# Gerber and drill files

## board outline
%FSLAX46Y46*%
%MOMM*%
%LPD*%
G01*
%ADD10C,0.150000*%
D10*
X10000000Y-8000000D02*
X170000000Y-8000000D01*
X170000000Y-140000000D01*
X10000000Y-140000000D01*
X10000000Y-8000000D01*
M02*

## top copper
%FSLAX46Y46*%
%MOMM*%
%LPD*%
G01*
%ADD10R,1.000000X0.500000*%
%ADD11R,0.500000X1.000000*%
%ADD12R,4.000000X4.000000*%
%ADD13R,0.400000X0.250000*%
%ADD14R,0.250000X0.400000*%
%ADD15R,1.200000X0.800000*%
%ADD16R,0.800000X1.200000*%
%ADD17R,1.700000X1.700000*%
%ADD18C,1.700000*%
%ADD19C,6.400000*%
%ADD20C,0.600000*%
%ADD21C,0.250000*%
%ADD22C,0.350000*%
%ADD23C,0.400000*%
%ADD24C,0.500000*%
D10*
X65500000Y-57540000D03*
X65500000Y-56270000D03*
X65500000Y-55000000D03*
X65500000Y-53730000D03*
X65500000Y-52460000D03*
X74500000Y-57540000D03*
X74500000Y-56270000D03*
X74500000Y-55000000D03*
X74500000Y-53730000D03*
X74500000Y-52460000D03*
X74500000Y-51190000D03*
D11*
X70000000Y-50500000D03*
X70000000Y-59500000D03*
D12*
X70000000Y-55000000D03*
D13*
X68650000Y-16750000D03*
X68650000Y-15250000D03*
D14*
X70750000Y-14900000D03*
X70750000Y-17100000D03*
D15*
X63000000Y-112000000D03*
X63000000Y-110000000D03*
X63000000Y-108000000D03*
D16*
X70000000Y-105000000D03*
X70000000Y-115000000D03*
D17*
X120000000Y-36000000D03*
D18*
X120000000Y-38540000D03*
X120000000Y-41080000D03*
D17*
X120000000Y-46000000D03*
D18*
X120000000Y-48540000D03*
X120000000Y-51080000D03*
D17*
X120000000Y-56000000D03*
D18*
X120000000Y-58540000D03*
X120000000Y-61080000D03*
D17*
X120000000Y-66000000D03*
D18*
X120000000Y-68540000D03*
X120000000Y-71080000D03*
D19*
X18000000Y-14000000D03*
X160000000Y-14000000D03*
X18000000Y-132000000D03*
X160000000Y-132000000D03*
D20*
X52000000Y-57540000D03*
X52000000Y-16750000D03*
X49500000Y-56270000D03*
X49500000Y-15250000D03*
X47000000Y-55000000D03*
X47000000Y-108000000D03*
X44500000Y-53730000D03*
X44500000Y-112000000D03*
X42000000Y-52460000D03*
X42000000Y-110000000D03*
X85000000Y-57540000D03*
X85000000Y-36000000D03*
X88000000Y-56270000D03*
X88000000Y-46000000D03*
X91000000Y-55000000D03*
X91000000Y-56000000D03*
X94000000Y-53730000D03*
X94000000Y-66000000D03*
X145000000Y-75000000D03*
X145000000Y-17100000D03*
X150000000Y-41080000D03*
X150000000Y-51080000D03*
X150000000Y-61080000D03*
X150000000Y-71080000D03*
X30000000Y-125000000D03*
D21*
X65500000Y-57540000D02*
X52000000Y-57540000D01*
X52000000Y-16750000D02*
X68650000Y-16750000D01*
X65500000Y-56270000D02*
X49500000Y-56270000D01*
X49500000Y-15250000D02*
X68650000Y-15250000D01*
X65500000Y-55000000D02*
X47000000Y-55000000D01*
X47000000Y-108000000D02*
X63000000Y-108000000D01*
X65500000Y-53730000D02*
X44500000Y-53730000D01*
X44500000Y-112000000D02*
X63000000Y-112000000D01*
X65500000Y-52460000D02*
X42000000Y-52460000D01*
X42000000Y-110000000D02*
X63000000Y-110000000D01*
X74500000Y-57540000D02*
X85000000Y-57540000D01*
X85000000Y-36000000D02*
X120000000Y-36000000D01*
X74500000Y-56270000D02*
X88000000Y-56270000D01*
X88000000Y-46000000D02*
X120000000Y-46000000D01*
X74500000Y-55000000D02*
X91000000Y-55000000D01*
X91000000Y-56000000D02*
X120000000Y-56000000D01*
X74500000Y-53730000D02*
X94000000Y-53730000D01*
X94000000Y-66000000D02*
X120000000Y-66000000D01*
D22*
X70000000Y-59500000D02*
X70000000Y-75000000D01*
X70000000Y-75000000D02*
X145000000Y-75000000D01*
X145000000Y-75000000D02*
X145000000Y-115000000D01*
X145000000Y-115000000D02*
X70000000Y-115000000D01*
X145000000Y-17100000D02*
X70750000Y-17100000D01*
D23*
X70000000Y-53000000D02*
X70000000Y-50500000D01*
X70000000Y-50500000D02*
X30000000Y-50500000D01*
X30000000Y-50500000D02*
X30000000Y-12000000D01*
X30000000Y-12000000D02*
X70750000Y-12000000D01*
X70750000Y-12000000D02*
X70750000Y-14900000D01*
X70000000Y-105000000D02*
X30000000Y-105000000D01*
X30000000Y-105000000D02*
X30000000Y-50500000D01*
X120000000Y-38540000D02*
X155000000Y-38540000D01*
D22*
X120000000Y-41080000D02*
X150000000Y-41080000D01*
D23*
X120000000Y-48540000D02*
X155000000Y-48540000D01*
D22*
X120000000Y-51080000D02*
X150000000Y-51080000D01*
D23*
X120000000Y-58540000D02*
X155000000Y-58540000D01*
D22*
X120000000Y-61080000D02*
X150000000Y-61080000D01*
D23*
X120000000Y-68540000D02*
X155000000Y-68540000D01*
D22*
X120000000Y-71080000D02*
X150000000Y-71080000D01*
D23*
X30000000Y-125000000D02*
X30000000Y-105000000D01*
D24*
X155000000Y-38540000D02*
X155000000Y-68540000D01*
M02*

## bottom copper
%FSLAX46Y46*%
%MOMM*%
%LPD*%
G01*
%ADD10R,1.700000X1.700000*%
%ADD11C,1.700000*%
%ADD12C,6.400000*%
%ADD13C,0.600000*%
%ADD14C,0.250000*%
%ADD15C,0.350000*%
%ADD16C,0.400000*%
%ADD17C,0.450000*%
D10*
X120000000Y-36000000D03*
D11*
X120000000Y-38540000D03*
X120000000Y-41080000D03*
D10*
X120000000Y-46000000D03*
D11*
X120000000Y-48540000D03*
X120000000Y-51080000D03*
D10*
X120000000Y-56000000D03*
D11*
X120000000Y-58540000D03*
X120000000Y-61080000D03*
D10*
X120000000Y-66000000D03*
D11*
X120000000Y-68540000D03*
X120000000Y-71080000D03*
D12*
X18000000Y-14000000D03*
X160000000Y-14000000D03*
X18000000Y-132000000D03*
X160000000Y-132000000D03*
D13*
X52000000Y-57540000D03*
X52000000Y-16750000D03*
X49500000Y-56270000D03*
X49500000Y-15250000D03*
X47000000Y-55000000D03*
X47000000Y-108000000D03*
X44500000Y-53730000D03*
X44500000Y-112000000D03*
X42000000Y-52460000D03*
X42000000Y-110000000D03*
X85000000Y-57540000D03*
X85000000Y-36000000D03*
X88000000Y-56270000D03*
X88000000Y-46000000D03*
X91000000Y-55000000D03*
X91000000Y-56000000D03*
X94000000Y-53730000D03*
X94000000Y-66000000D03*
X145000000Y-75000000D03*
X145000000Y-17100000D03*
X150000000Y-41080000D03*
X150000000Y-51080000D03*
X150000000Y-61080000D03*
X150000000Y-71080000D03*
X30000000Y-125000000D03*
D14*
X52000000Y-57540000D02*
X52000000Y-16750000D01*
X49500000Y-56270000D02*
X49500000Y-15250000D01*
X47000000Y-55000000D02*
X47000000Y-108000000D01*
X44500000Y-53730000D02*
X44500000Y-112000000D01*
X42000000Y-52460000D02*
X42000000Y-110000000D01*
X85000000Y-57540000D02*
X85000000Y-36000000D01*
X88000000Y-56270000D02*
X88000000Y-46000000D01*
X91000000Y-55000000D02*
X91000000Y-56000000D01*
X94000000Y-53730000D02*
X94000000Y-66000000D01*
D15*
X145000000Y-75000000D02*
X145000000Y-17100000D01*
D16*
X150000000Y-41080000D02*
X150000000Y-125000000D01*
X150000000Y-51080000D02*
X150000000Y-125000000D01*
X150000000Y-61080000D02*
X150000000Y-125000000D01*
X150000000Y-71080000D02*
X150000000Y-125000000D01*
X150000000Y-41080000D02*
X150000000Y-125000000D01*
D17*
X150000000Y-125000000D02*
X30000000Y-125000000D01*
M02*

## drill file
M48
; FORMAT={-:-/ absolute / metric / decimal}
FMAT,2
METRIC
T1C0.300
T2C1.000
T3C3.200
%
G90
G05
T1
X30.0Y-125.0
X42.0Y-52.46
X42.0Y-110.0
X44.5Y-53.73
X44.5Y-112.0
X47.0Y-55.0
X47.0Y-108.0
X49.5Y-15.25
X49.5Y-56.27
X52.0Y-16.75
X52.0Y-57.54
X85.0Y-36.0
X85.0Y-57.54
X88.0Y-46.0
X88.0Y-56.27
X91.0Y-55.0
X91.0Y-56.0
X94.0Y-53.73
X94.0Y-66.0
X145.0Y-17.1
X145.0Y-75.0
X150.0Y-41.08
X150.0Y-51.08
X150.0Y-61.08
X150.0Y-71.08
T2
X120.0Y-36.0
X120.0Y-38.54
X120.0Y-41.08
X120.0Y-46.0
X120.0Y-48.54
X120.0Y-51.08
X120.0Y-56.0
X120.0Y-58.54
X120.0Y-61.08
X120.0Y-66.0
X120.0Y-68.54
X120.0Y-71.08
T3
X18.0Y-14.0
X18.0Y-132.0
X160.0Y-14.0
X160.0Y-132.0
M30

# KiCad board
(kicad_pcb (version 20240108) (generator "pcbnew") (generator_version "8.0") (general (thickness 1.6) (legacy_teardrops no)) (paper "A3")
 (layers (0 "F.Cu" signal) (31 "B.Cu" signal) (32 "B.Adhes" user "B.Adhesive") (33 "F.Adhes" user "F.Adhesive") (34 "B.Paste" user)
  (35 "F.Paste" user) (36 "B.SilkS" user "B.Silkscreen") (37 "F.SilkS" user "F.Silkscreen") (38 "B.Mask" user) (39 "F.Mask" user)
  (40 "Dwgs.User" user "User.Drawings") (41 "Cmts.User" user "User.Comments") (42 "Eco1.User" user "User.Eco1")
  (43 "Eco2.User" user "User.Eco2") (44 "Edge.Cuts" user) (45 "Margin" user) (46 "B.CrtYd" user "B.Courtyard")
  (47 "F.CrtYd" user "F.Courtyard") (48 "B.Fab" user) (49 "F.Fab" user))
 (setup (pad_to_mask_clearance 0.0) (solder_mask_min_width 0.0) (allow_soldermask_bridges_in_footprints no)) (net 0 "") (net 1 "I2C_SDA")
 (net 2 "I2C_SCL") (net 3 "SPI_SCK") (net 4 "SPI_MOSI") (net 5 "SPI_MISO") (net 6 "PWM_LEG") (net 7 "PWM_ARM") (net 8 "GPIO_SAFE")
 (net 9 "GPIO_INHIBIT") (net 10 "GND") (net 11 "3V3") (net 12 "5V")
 (gr_rect (start 10 8) (end 170 140) (stroke (width 0.15) (type solid)) (fill none) (layer "Edge.Cuts"))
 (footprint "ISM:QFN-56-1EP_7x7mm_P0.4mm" (layer "F.Cu") (at 70 55)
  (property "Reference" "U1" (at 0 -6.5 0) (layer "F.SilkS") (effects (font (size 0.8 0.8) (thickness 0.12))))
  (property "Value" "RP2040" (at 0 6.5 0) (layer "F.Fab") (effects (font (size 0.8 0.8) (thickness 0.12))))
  (pad "1" smd rect (at -4.5 2.54) (size 1.0 0.5) (layers "F.Cu" "F.Paste" "F.Mask") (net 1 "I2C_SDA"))
  (pad "2" smd rect (at -4.5 1.27) (size 1.0 0.5) (layers "F.Cu" "F.Paste" "F.Mask") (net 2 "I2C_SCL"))
  (pad "3" smd rect (at -4.5 0) (size 1.0 0.5) (layers "F.Cu" "F.Paste" "F.Mask") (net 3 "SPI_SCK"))
  (pad "4" smd rect (at -4.5 -1.27) (size 1.0 0.5) (layers "F.Cu" "F.Paste" "F.Mask") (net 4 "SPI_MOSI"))
  (pad "5" smd rect (at -4.5 -2.54) (size 1.0 0.5) (layers "F.Cu" "F.Paste" "F.Mask") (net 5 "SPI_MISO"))
  (pad "6" smd rect (at 4.5 2.54) (size 1.0 0.5) (layers "F.Cu" "F.Paste" "F.Mask") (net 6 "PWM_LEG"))
  (pad "7" smd rect (at 4.5 1.27) (size 1.0 0.5) (layers "F.Cu" "F.Paste" "F.Mask") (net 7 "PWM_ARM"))
  (pad "8" smd rect (at 4.5 0) (size 1.0 0.5) (layers "F.Cu" "F.Paste" "F.Mask") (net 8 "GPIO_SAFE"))
  (pad "9" smd rect (at 4.5 -1.27) (size 1.0 0.5) (layers "F.Cu" "F.Paste" "F.Mask") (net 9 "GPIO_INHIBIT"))
  (pad "12" smd rect (at 4.5 -2.54) (size 1.0 0.5) (layers "F.Cu" "F.Paste" "F.Mask"))
  (pad "13" smd rect (at 4.5 -3.81) (size 1.0 0.5) (layers "F.Cu" "F.Paste" "F.Mask"))
  (pad "10" smd rect (at 0 -4.5) (size 0.5 1.0) (layers "F.Cu" "F.Paste" "F.Mask") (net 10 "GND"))
  (pad "11" smd rect (at 0 4.5) (size 0.5 1.0) (layers "F.Cu" "F.Paste" "F.Mask") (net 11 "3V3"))
  (pad "EP" smd rect (at 0 0) (size 4 4) (layers "F.Cu" "F.Paste" "F.Mask") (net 10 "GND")))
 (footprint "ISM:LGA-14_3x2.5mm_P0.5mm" (layer "F.Cu") (at 70 16)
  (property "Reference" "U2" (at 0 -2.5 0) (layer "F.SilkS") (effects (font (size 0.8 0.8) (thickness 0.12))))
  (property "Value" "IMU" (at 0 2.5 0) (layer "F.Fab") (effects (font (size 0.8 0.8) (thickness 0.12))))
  (pad "1" smd rect (at -1.35 0.75) (size 0.4 0.25) (layers "F.Cu" "F.Paste" "F.Mask") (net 1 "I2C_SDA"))
  (pad "2" smd rect (at -1.35 -0.75) (size 0.4 0.25) (layers "F.Cu" "F.Paste" "F.Mask") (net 2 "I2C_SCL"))
  (pad "3" smd rect (at 0.75 -1.1) (size 0.25 0.4) (layers "F.Cu" "F.Paste" "F.Mask") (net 10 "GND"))
  (pad "4" smd rect (at 0.75 1.1) (size 0.25 0.4) (layers "F.Cu" "F.Paste" "F.Mask") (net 11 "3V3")))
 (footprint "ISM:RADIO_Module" (layer "F.Cu") (at 70 110)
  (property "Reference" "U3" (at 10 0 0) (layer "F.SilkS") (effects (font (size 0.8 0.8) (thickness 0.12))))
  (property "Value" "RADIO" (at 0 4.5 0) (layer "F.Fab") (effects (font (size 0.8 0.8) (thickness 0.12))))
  (pad "1" smd rect (at -7 2) (size 1.2 0.8) (layers "F.Cu" "F.Paste" "F.Mask") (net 4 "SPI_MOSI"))
  (pad "2" smd rect (at -7 0) (size 1.2 0.8) (layers "F.Cu" "F.Paste" "F.Mask") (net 5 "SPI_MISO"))
  (pad "3" smd rect (at -7 -2) (size 1.2 0.8) (layers "F.Cu" "F.Paste" "F.Mask") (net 3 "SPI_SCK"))
  (pad "4" smd rect (at 0 -5) (size 0.8 1.2) (layers "F.Cu" "F.Paste" "F.Mask") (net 10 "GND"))
  (pad "5" smd rect (at 0 5) (size 0.8 1.2) (layers "F.Cu" "F.Paste" "F.Mask") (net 11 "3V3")))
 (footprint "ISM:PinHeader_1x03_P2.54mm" (layer "F.Cu") (at 120 36)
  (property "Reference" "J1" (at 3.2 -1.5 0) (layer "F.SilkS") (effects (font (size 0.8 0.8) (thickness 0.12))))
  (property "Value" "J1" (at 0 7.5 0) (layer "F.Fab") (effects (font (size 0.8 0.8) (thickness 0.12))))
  (pad "1" thru_hole rect (at 0 0) (size 1.7 1.7) (drill 1.0) (layers "*.Cu" "*.Mask") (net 6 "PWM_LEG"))
  (pad "2" thru_hole circle (at 0 2.54) (size 1.7 1.7) (drill 1.0) (layers "*.Cu" "*.Mask") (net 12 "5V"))
  (pad "3" thru_hole circle (at 0 5.08) (size 1.7 1.7) (drill 1.0) (layers "*.Cu" "*.Mask") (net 10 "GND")))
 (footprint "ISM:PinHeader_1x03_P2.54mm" (layer "F.Cu") (at 120 46)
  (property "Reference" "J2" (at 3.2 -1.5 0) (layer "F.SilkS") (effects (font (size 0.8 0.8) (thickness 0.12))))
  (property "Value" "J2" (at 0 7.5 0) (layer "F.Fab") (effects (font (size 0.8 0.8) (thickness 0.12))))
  (pad "1" thru_hole rect (at 0 0) (size 1.7 1.7) (drill 1.0) (layers "*.Cu" "*.Mask") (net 7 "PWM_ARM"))
  (pad "2" thru_hole circle (at 0 2.54) (size 1.7 1.7) (drill 1.0) (layers "*.Cu" "*.Mask") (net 12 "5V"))
  (pad "3" thru_hole circle (at 0 5.08) (size 1.7 1.7) (drill 1.0) (layers "*.Cu" "*.Mask") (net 10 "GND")))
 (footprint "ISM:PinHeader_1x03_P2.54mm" (layer "F.Cu") (at 120 56)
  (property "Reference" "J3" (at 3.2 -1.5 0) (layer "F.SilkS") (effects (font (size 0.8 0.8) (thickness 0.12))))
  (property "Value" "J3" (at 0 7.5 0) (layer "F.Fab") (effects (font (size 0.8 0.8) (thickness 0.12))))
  (pad "1" thru_hole rect (at 0 0) (size 1.7 1.7) (drill 1.0) (layers "*.Cu" "*.Mask") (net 8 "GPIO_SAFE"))
  (pad "2" thru_hole circle (at 0 2.54) (size 1.7 1.7) (drill 1.0) (layers "*.Cu" "*.Mask") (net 12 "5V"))
  (pad "3" thru_hole circle (at 0 5.08) (size 1.7 1.7) (drill 1.0) (layers "*.Cu" "*.Mask") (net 10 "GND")))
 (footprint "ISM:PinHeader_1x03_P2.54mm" (layer "F.Cu") (at 120 66)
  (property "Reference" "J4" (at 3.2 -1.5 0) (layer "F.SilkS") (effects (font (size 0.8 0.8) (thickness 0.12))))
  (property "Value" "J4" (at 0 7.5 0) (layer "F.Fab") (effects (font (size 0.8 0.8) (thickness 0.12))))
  (pad "1" thru_hole rect (at 0 0) (size 1.7 1.7) (drill 1.0) (layers "*.Cu" "*.Mask") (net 9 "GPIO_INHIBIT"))
  (pad "2" thru_hole circle (at 0 2.54) (size 1.7 1.7) (drill 1.0) (layers "*.Cu" "*.Mask") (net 12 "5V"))
  (pad "3" thru_hole circle (at 0 5.08) (size 1.7 1.7) (drill 1.0) (layers "*.Cu" "*.Mask") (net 10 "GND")))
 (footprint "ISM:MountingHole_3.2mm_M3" (layer "F.Cu") (at 18 14)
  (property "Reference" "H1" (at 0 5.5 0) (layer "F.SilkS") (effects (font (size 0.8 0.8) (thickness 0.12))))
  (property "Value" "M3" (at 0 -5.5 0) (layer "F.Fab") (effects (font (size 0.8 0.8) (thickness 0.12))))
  (pad "" thru_hole circle (at 0 0) (size 6.4 6.4) (drill 3.2) (layers "*.Cu" "*.Mask")))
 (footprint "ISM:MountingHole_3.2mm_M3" (layer "F.Cu") (at 160 14)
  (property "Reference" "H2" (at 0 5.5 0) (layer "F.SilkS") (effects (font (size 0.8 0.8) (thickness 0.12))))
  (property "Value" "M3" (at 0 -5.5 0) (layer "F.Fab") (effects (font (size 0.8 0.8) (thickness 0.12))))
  (pad "" thru_hole circle (at 0 0) (size 6.4 6.4) (drill 3.2) (layers "*.Cu" "*.Mask")))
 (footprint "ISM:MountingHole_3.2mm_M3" (layer "F.Cu") (at 18 132)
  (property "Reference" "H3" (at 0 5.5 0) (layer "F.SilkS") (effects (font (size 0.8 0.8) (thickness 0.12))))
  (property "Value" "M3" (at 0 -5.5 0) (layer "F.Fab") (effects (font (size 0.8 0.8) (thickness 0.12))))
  (pad "" thru_hole circle (at 0 0) (size 6.4 6.4) (drill 3.2) (layers "*.Cu" "*.Mask")))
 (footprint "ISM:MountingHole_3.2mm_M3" (layer "F.Cu") (at 160 132)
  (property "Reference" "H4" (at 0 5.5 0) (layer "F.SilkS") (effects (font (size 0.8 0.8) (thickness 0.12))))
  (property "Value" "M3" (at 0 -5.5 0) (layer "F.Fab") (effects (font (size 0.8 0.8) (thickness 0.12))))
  (pad "" thru_hole circle (at 0 0) (size 6.4 6.4) (drill 3.2) (layers "*.Cu" "*.Mask")))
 (segment (start 65.5 57.54) (end 52.0 57.54) (width 0.25) (layer "F.Cu") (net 1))
 (segment (start 52.0 57.54) (end 52.0 16.75) (width 0.25) (layer "B.Cu") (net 1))
 (segment (start 52.0 16.75) (end 68.65 16.75) (width 0.25) (layer "F.Cu") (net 1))
 (segment (start 65.5 56.27) (end 49.5 56.27) (width 0.25) (layer "F.Cu") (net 2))
 (segment (start 49.5 56.27) (end 49.5 15.25) (width 0.25) (layer "B.Cu") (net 2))
 (segment (start 49.5 15.25) (end 68.65 15.25) (width 0.25) (layer "F.Cu") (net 2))
 (segment (start 65.5 55) (end 47.0 55) (width 0.25) (layer "F.Cu") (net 3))
 (segment (start 47.0 55) (end 47.0 108) (width 0.25) (layer "B.Cu") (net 3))
 (segment (start 47.0 108) (end 63 108) (width 0.25) (layer "F.Cu") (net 3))
 (segment (start 65.5 53.73) (end 44.5 53.73) (width 0.25) (layer "F.Cu") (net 4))
 (segment (start 44.5 53.73) (end 44.5 112) (width 0.25) (layer "B.Cu") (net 4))
 (segment (start 44.5 112) (end 63 112) (width 0.25) (layer "F.Cu") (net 4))
 (segment (start 65.5 52.46) (end 42.0 52.46) (width 0.25) (layer "F.Cu") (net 5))
 (segment (start 42.0 52.46) (end 42.0 110) (width 0.25) (layer "B.Cu") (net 5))
 (segment (start 42.0 110) (end 63 110) (width 0.25) (layer "F.Cu") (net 5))
 (segment (start 74.5 57.54) (end 85 57.54) (width 0.25) (layer "F.Cu") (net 6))
 (segment (start 85 57.54) (end 85 36) (width 0.25) (layer "B.Cu") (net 6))
 (segment (start 85 36) (end 120 36) (width 0.25) (layer "F.Cu") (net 6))
 (segment (start 74.5 56.27) (end 88 56.27) (width 0.25) (layer "F.Cu") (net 7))
 (segment (start 88 56.27) (end 88 46) (width 0.25) (layer "B.Cu") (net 7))
 (segment (start 88 46) (end 120 46) (width 0.25) (layer "F.Cu") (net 7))
 (segment (start 74.5 55) (end 91 55) (width 0.25) (layer "F.Cu") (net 8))
 (segment (start 91 55) (end 91 56) (width 0.25) (layer "B.Cu") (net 8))
 (segment (start 91 56) (end 120 56) (width 0.25) (layer "F.Cu") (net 8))
 (segment (start 74.5 53.73) (end 94 53.73) (width 0.25) (layer "F.Cu") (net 9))
 (segment (start 94 53.73) (end 94 66) (width 0.25) (layer "B.Cu") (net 9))
 (segment (start 94 66) (end 120 66) (width 0.25) (layer "F.Cu") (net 9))
 (segment (start 70 59.5) (end 70 75) (width 0.35) (layer "F.Cu") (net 11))
 (segment (start 70 75) (end 145 75) (width 0.35) (layer "F.Cu") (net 11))
 (segment (start 145 75) (end 145 115) (width 0.35) (layer "F.Cu") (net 11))
 (segment (start 145 115) (end 70 115) (width 0.35) (layer "F.Cu") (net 11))
 (segment (start 145 75) (end 145 17.1) (width 0.35) (layer "B.Cu") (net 11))
 (segment (start 145 17.1) (end 70.75 17.1) (width 0.35) (layer "F.Cu") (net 11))
 (segment (start 70 53) (end 70 50.5) (width 0.4) (layer "F.Cu") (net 10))
 (segment (start 70 50.5) (end 30 50.5) (width 0.4) (layer "F.Cu") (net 10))
 (segment (start 30 50.5) (end 30 12) (width 0.4) (layer "F.Cu") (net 10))
 (segment (start 30 12) (end 70.75 12) (width 0.4) (layer "F.Cu") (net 10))
 (segment (start 70.75 12) (end 70.75 14.9) (width 0.4) (layer "F.Cu") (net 10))
 (segment (start 70 105) (end 30 105) (width 0.4) (layer "F.Cu") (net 10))
 (segment (start 30 105) (end 30 50.5) (width 0.4) (layer "F.Cu") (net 10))
 (segment (start 120 38.54) (end 155 38.54) (width 0.4) (layer "F.Cu") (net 12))
 (segment (start 120 41.08) (end 150 41.08) (width 0.35) (layer "F.Cu") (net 10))
 (segment (start 150 41.08) (end 150 125) (width 0.4) (layer "B.Cu") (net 10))
 (segment (start 120 48.54) (end 155 48.54) (width 0.4) (layer "F.Cu") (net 12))
 (segment (start 120 51.08) (end 150 51.08) (width 0.35) (layer "F.Cu") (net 10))
 (segment (start 150 51.08) (end 150 125) (width 0.4) (layer "B.Cu") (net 10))
 (segment (start 120 58.54) (end 155 58.54) (width 0.4) (layer "F.Cu") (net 12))
 (segment (start 120 61.08) (end 150 61.08) (width 0.35) (layer "F.Cu") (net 10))
 (segment (start 150 61.08) (end 150 125) (width 0.4) (layer "B.Cu") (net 10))
 (segment (start 120 68.54) (end 155 68.54) (width 0.4) (layer "F.Cu") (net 12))
 (segment (start 120 71.08) (end 150 71.08) (width 0.35) (layer "F.Cu") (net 10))
 (segment (start 150 71.08) (end 150 125) (width 0.4) (layer "B.Cu") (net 10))
 (segment (start 150 41.08) (end 150 125) (width 0.4) (layer "B.Cu") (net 10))
 (segment (start 150 125) (end 30 125) (width 0.45) (layer "B.Cu") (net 10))
 (segment (start 30 125) (end 30 105) (width 0.4) (layer "F.Cu") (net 10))
 (segment (start 155 38.54) (end 155 68.54) (width 0.5) (layer "F.Cu") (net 12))
 (via (at 52.0 57.54) (size 0.6) (drill 0.3) (layers "F.Cu" "B.Cu") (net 1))
 (via (at 52.0 16.75) (size 0.6) (drill 0.3) (layers "F.Cu" "B.Cu") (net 1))
 (via (at 49.5 56.27) (size 0.6) (drill 0.3) (layers "F.Cu" "B.Cu") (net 2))
 (via (at 49.5 15.25) (size 0.6) (drill 0.3) (layers "F.Cu" "B.Cu") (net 2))
 (via (at 47.0 55) (size 0.6) (drill 0.3) (layers "F.Cu" "B.Cu") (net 3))
 (via (at 47.0 108) (size 0.6) (drill 0.3) (layers "F.Cu" "B.Cu") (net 3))
 (via (at 44.5 53.73) (size 0.6) (drill 0.3) (layers "F.Cu" "B.Cu") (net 4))
 (via (at 44.5 112) (size 0.6) (drill 0.3) (layers "F.Cu" "B.Cu") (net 4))
 (via (at 42.0 52.46) (size 0.6) (drill 0.3) (layers "F.Cu" "B.Cu") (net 5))
 (via (at 42.0 110) (size 0.6) (drill 0.3) (layers "F.Cu" "B.Cu") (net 5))
 (via (at 85 57.54) (size 0.6) (drill 0.3) (layers "F.Cu" "B.Cu") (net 6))
 (via (at 85 36) (size 0.6) (drill 0.3) (layers "F.Cu" "B.Cu") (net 6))
 (via (at 88 56.27) (size 0.6) (drill 0.3) (layers "F.Cu" "B.Cu") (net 7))
 (via (at 88 46) (size 0.6) (drill 0.3) (layers "F.Cu" "B.Cu") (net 7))
 (via (at 91 55) (size 0.6) (drill 0.3) (layers "F.Cu" "B.Cu") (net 8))
 (via (at 91 56) (size 0.6) (drill 0.3) (layers "F.Cu" "B.Cu") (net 8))
 (via (at 94 53.73) (size 0.6) (drill 0.3) (layers "F.Cu" "B.Cu") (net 9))
 (via (at 94 66) (size 0.6) (drill 0.3) (layers "F.Cu" "B.Cu") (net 9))
 (via (at 145 75) (size 0.6) (drill 0.3) (layers "F.Cu" "B.Cu") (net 11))
 (via (at 145 17.1) (size 0.6) (drill 0.3) (layers "F.Cu" "B.Cu") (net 11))
 (via (at 150 41.08) (size 0.6) (drill 0.3) (layers "F.Cu" "B.Cu") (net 10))
 (via (at 150 51.08) (size 0.6) (drill 0.3) (layers "F.Cu" "B.Cu") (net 10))
 (via (at 150 61.08) (size 0.6) (drill 0.3) (layers "F.Cu" "B.Cu") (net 10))
 (via (at 150 71.08) (size 0.6) (drill 0.3) (layers "F.Cu" "B.Cu") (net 10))
 (via (at 30 125) (size 0.6) (drill 0.3) (layers "F.Cu" "B.Cu") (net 10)))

